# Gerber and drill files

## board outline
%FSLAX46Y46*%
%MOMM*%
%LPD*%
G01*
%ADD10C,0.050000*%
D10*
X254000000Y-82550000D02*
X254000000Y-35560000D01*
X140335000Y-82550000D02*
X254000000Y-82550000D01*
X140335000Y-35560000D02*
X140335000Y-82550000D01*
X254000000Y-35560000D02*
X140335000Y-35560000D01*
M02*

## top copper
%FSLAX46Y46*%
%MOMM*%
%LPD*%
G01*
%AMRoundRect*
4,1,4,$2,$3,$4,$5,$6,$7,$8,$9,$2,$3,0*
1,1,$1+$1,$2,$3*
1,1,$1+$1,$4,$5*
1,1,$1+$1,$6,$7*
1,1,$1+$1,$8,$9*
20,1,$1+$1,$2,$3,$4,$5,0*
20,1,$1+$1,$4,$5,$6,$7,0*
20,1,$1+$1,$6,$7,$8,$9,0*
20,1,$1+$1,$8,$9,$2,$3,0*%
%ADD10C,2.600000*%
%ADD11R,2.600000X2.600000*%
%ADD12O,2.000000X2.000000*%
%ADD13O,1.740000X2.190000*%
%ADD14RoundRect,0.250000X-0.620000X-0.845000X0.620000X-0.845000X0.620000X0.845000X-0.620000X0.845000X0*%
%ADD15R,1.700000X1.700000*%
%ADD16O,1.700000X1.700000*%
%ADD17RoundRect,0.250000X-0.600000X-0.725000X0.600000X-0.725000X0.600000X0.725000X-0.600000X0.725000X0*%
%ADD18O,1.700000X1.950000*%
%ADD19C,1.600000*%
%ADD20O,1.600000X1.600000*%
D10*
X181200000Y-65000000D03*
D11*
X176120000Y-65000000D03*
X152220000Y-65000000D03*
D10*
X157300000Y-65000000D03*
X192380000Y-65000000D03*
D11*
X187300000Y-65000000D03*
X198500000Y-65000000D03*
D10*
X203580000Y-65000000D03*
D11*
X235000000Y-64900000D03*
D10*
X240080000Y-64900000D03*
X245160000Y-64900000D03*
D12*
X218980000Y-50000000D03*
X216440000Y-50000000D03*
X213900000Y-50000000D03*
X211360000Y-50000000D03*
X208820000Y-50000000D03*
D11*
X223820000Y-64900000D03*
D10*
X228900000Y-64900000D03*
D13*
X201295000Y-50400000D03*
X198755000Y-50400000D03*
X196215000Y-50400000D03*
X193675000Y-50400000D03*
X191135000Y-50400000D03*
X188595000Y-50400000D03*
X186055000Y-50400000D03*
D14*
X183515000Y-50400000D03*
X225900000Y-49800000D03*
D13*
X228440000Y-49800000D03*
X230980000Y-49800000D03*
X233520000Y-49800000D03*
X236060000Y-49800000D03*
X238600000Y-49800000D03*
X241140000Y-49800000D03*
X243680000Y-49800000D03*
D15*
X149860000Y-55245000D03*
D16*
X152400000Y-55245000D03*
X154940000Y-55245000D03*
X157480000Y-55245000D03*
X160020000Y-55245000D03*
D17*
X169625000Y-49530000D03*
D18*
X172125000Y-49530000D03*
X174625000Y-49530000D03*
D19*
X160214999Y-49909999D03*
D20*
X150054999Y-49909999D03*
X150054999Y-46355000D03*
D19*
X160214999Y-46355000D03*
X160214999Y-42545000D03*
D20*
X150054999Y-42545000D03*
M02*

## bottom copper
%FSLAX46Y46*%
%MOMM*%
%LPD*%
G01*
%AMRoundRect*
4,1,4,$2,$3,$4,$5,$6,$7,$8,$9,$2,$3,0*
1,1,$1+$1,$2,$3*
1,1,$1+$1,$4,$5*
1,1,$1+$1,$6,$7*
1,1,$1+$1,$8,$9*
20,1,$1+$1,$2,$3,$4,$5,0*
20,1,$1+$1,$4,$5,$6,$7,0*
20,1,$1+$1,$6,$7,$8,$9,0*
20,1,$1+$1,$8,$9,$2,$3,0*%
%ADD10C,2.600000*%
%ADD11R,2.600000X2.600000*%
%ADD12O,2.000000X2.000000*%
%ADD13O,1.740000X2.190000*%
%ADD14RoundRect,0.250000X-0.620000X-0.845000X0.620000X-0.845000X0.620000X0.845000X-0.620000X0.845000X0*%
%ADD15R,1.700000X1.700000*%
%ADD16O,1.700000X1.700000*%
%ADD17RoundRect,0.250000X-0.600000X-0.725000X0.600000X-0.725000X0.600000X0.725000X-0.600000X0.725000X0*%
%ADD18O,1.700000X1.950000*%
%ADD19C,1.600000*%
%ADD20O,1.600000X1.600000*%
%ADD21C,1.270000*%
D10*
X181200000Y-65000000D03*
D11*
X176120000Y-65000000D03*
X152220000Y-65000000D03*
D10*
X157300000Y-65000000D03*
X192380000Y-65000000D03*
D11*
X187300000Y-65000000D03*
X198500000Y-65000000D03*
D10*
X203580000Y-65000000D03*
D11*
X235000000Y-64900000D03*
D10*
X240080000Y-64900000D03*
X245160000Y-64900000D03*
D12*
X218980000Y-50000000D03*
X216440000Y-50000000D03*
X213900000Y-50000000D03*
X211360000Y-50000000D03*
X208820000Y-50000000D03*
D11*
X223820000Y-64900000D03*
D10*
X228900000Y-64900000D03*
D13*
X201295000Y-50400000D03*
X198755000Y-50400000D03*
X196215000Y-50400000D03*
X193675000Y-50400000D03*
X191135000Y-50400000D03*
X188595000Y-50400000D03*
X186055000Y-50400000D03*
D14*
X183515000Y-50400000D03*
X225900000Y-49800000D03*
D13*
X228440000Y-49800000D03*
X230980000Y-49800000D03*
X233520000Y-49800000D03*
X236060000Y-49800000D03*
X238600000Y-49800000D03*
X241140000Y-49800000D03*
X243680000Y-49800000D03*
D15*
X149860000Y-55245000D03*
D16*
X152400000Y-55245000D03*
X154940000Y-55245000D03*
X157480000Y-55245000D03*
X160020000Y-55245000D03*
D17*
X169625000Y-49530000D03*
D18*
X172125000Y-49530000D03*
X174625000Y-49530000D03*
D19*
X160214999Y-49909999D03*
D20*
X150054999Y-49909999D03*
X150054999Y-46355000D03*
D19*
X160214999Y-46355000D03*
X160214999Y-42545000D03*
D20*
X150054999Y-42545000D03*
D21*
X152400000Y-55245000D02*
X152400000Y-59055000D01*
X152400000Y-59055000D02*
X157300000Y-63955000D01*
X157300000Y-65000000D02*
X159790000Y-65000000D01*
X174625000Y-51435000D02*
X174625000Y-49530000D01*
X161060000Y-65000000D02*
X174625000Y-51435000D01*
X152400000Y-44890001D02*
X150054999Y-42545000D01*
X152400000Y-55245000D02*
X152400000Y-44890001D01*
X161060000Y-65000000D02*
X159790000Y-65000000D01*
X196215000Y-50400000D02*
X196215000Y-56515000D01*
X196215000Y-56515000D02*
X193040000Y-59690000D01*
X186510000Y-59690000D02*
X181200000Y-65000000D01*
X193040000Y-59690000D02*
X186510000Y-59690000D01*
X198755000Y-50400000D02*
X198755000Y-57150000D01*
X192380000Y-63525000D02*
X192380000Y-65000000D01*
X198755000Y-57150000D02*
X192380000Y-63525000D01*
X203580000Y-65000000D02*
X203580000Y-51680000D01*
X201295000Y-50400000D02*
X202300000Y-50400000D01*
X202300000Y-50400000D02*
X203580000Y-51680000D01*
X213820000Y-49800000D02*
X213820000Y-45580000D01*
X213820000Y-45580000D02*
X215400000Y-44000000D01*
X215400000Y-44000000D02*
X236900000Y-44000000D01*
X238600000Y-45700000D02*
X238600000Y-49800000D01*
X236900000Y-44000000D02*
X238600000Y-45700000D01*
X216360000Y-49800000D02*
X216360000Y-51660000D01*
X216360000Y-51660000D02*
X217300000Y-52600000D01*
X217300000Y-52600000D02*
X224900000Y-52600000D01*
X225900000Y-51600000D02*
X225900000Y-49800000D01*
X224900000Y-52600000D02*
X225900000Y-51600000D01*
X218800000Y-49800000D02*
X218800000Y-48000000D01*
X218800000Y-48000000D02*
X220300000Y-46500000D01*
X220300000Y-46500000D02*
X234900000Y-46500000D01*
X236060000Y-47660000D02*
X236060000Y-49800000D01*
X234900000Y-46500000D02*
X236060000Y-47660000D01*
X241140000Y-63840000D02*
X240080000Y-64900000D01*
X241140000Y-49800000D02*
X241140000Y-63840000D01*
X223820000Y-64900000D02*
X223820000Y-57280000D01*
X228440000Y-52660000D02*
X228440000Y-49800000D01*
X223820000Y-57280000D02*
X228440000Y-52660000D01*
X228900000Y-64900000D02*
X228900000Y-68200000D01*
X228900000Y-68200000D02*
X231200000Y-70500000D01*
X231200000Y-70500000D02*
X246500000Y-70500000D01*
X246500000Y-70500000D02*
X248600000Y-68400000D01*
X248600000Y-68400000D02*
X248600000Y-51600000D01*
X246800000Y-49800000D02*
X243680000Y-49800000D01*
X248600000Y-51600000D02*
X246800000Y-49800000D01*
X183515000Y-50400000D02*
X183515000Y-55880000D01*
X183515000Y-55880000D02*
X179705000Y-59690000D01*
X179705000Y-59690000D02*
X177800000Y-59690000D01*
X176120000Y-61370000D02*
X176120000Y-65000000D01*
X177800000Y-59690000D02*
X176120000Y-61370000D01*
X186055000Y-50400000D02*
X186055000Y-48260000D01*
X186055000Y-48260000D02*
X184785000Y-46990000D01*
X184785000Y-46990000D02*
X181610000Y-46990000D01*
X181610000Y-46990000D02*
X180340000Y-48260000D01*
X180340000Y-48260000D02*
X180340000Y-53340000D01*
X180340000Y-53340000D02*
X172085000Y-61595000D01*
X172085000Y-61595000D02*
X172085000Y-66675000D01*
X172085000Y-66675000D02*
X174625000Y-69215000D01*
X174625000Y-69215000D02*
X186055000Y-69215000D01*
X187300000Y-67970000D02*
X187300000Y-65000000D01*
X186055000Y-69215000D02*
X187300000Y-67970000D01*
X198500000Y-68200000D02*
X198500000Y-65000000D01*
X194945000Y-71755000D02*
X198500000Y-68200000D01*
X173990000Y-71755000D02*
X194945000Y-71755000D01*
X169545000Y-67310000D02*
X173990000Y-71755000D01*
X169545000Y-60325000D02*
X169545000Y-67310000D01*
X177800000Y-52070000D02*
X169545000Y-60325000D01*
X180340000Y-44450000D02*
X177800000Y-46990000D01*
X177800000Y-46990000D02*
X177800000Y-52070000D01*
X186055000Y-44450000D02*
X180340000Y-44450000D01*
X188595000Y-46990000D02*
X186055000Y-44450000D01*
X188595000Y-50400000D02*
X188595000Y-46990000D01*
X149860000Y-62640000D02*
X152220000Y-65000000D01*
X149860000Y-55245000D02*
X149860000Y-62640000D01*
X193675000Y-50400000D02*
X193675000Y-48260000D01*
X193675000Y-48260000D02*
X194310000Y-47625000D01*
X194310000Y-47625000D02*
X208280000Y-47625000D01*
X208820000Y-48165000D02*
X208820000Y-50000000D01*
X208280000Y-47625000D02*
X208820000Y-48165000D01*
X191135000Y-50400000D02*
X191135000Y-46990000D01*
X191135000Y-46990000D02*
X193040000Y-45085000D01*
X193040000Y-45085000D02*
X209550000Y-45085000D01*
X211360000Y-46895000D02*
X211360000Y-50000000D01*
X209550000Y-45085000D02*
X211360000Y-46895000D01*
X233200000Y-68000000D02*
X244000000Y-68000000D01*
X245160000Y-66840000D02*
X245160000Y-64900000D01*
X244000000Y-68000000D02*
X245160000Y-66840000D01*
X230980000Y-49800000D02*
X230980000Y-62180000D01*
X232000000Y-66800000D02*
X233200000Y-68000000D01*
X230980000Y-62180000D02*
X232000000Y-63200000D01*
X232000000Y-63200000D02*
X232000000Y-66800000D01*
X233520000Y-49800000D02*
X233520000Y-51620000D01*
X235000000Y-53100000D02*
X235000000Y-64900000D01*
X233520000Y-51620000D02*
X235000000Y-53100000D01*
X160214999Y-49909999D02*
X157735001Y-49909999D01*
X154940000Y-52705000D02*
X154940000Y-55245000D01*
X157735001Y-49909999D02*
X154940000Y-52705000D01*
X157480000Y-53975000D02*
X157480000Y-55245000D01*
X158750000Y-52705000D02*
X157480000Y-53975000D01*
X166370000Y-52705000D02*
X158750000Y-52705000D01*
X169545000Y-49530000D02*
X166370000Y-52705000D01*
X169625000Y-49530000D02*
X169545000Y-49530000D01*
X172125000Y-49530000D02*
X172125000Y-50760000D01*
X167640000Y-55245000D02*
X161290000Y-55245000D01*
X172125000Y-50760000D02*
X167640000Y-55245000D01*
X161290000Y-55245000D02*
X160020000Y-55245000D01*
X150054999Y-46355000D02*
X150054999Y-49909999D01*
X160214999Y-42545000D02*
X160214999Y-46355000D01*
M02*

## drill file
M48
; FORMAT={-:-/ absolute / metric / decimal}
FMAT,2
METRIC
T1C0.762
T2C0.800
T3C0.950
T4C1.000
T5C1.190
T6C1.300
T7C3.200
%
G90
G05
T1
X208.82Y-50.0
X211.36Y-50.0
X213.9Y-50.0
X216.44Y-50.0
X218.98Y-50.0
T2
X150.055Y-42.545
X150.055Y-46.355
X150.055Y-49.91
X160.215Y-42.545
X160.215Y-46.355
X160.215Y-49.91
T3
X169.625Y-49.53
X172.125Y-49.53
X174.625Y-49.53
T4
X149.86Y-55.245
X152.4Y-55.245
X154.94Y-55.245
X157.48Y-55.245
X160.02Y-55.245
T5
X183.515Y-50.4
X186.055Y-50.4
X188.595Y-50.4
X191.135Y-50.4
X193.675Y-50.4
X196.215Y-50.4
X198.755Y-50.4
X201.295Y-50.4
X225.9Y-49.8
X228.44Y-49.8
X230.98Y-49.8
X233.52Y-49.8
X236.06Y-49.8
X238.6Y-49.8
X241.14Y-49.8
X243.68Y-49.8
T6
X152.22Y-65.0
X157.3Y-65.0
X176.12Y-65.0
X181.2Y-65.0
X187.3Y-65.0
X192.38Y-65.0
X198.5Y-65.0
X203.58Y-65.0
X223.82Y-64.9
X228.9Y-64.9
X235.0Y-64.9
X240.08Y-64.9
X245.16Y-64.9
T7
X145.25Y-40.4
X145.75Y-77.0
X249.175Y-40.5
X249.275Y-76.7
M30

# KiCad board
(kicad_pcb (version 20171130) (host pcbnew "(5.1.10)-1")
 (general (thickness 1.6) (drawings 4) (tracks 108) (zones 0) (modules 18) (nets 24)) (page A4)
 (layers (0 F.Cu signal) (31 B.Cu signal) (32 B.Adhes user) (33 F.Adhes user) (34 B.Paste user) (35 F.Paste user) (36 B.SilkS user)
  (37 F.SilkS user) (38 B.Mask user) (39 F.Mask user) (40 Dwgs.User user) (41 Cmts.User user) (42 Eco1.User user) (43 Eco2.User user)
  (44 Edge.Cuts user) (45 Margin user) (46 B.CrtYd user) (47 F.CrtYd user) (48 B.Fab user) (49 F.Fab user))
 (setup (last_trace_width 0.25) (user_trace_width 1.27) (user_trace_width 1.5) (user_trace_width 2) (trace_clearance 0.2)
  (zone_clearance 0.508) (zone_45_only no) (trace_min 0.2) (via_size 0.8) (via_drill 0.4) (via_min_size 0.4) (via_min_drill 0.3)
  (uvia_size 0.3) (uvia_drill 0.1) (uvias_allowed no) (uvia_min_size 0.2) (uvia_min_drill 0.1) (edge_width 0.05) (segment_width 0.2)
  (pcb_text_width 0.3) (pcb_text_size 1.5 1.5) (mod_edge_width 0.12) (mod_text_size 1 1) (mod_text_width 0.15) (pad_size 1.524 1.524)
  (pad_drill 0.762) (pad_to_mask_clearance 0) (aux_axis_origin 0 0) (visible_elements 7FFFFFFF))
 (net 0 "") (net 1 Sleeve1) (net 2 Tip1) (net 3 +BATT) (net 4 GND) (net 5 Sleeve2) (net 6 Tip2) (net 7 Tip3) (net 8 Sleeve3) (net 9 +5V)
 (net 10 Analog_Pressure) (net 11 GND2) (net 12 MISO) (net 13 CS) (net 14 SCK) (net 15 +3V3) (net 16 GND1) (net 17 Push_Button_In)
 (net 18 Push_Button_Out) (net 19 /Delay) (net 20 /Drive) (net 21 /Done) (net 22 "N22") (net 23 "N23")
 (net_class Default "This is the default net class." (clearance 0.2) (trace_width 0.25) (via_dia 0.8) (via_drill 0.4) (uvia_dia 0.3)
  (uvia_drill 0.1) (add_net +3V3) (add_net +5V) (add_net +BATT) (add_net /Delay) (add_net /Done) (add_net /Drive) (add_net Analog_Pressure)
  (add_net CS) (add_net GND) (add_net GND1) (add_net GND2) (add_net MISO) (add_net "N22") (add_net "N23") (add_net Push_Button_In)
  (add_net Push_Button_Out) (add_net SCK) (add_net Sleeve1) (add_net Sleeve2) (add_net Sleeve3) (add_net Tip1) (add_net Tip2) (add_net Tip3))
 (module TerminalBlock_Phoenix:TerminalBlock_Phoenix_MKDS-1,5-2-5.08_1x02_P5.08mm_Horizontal (layer F.Cu) (at 176.12 65)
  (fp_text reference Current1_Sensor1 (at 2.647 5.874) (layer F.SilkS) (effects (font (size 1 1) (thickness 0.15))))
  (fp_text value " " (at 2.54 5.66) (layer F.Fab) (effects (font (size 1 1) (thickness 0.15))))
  (pad 2 thru_hole circle (at 5.08 0) (size 2.6 2.6) (drill 1.3) (layers *.Cu *.Mask) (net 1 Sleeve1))
  (pad 1 thru_hole rect (at 0 0) (size 2.6 2.6) (drill 1.3) (layers *.Cu *.Mask) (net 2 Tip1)))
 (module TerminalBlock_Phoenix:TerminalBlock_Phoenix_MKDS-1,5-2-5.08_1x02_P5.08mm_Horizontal (layer F.Cu) (at 152.22 65)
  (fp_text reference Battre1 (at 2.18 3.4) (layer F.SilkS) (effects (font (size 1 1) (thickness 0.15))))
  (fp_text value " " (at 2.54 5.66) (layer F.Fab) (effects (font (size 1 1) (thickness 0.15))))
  (pad 1 thru_hole rect (at 0 0) (size 2.6 2.6) (drill 1.3) (layers *.Cu *.Mask) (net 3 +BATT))
  (pad 2 thru_hole circle (at 5.08 0) (size 2.6 2.6) (drill 1.3) (layers *.Cu *.Mask) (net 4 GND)))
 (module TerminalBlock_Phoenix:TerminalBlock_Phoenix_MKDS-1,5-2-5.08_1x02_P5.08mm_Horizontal (layer F.Cu) (at 187.3 65)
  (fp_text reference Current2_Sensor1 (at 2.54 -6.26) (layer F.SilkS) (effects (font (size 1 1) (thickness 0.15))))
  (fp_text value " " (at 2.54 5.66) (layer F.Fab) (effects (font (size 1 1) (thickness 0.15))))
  (pad 2 thru_hole circle (at 5.08 0) (size 2.6 2.6) (drill 1.3) (layers *.Cu *.Mask) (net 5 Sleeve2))
  (pad 1 thru_hole rect (at 0 0) (size 2.6 2.6) (drill 1.3) (layers *.Cu *.Mask) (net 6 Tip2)))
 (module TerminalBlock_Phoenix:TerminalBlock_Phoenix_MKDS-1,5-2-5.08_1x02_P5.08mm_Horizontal (layer F.Cu) (at 198.5 65)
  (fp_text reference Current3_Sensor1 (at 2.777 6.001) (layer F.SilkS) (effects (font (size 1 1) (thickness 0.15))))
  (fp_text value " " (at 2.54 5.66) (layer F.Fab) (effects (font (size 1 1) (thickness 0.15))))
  (pad 1 thru_hole rect (at 0 0) (size 2.6 2.6) (drill 1.3) (layers *.Cu *.Mask) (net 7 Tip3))
  (pad 2 thru_hole circle (at 5.08 0) (size 2.6 2.6) (drill 1.3) (layers *.Cu *.Mask) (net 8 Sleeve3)))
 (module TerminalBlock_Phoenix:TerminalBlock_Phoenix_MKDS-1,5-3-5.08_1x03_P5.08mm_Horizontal (layer F.Cu) (at 235 64.9)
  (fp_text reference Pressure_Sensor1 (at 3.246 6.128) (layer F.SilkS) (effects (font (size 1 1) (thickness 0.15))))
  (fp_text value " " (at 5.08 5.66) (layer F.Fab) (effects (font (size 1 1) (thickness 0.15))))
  (pad 1 thru_hole rect (at 0 0) (size 2.6 2.6) (drill 1.3) (layers *.Cu *.Mask) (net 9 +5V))
  (pad 2 thru_hole circle (at 5.08 0) (size 2.6 2.6) (drill 1.3) (layers *.Cu *.Mask) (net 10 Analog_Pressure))
  (pad 3 thru_hole circle (at 10.16 0) (size 2.6 2.6) (drill 1.3) (layers *.Cu *.Mask) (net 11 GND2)))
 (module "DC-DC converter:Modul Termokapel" (layer F.Cu) (at 213.9 55.08)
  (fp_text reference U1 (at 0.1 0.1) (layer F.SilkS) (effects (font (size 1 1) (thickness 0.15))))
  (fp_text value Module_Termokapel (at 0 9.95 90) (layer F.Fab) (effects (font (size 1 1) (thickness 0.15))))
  (pad 5 thru_hole oval (at 5.08 -5.08) (size 2 2) (drill 0.762) (layers *.Cu *.Mask) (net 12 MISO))
  (pad 4 thru_hole oval (at 2.54 -5.08) (size 2 2) (drill 0.762) (layers *.Cu *.Mask) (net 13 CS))
  (pad 3 thru_hole oval (at 0 -5.08) (size 2 2) (drill 0.762) (layers *.Cu *.Mask) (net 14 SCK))
  (pad 2 thru_hole oval (at -2.54 -5.08) (size 2 2) (drill 0.762) (layers *.Cu *.Mask) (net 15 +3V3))
  (pad 1 thru_hole oval (at -5.08 -5.08) (size 2 2) (drill 0.762) (layers *.Cu *.Mask) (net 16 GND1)))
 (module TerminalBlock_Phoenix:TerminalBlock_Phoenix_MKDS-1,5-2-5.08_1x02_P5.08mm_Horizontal (layer F.Cu) (at 223.82 64.9)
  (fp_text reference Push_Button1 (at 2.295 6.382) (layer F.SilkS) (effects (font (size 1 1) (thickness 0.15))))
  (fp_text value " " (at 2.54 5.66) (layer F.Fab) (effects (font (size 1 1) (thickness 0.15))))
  (pad 1 thru_hole rect (at 0 0) (size 2.6 2.6) (drill 1.3) (layers *.Cu *.Mask) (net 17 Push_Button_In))
  (pad 2 thru_hole circle (at 5.08 0) (size 2.6 2.6) (drill 1.3) (layers *.Cu *.Mask) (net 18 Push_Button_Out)))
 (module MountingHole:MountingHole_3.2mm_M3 (layer F.Cu) (at 145.75 77)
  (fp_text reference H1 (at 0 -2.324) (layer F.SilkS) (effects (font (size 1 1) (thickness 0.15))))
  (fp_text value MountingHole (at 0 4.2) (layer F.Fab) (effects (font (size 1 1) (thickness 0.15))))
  (pad 1 np_thru_hole circle (at 0 0) (size 3.2 3.2) (drill 3.2) (layers *.Cu *.Mask)))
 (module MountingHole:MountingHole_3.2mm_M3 (layer F.Cu) (at 145.25 40.4)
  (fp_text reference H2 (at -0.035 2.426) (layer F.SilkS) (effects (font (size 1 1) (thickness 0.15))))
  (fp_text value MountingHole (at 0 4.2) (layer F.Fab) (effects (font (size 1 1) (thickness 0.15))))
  (pad 1 np_thru_hole circle (at 0 0) (size 3.2 3.2) (drill 3.2) (layers *.Cu *.Mask)))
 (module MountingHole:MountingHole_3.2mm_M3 (layer F.Cu) (at 249.275 76.7)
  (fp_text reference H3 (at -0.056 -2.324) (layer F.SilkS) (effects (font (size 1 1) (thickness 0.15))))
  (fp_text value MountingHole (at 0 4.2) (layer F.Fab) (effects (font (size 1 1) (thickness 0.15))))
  (pad 1 np_thru_hole circle (at 0 0) (size 3.2 3.2) (drill 3.2) (layers *.Cu *.Mask)))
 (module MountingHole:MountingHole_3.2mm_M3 (layer F.Cu) (at 249.175 40.5)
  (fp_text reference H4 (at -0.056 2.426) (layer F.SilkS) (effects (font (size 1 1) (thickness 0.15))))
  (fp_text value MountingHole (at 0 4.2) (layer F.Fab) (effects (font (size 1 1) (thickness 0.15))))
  (pad 1 np_thru_hole circle (at 0 0) (size 3.2 3.2) (drill 3.2) (layers *.Cu *.Mask)))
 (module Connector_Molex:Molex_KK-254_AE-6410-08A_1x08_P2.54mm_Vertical (layer F.Cu) (at 183.515 50.4)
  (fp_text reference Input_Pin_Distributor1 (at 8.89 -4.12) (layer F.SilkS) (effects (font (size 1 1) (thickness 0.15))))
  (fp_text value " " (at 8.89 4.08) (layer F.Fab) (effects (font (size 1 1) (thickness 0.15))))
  (pad 8 thru_hole oval (at 17.78 0) (size 1.74 2.19) (drill 1.19) (layers *.Cu *.Mask) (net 8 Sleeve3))
  (pad 7 thru_hole oval (at 15.24 0) (size 1.74 2.19) (drill 1.19) (layers *.Cu *.Mask) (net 5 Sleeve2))
  (pad 6 thru_hole oval (at 12.7 0) (size 1.74 2.19) (drill 1.19) (layers *.Cu *.Mask) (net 1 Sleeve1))
  (pad 5 thru_hole oval (at 10.16 0) (size 1.74 2.19) (drill 1.19) (layers *.Cu *.Mask) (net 16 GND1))
  (pad 4 thru_hole oval (at 7.62 0) (size 1.74 2.19) (drill 1.19) (layers *.Cu *.Mask) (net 15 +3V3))
  (pad 3 thru_hole oval (at 5.08 0) (size 1.74 2.19) (drill 1.19) (layers *.Cu *.Mask) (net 7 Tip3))
  (pad 2 thru_hole oval (at 2.54 0) (size 1.74 2.19) (drill 1.19) (layers *.Cu *.Mask) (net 6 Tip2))
  (pad 1 thru_hole roundrect (at 0 0) (size 1.74 2.19) (drill 1.19) (layers *.Cu *.Mask) (roundrect_rratio 0.143678) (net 2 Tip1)))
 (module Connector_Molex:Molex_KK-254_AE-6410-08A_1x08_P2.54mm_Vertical (layer F.Cu) (at 225.9 49.8)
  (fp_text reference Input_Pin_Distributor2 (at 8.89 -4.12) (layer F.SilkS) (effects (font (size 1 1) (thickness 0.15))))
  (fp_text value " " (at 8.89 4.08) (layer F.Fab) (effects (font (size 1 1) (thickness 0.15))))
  (pad 1 thru_hole roundrect (at 0 0) (size 1.74 2.19) (drill 1.19) (layers *.Cu *.Mask) (roundrect_rratio 0.143678) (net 13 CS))
  (pad 2 thru_hole oval (at 2.54 0) (size 1.74 2.19) (drill 1.19) (layers *.Cu *.Mask) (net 17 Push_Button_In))
  (pad 3 thru_hole oval (at 5.08 0) (size 1.74 2.19) (drill 1.19) (layers *.Cu *.Mask) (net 11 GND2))
  (pad 4 thru_hole oval (at 7.62 0) (size 1.74 2.19) (drill 1.19) (layers *.Cu *.Mask) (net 9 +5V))
  (pad 5 thru_hole oval (at 10.16 0) (size 1.74 2.19) (drill 1.19) (layers *.Cu *.Mask) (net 12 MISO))
  (pad 6 thru_hole oval (at 12.7 0) (size 1.74 2.19) (drill 1.19) (layers *.Cu *.Mask) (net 14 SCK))
  (pad 7 thru_hole oval (at 15.24 0) (size 1.74 2.19) (drill 1.19) (layers *.Cu *.Mask) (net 10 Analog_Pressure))
  (pad 8 thru_hole oval (at 17.78 0) (size 1.74 2.19) (drill 1.19) (layers *.Cu *.Mask) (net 18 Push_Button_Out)))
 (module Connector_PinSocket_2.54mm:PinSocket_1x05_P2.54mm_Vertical (layer F.Cu) (at 149.86 55.245 90)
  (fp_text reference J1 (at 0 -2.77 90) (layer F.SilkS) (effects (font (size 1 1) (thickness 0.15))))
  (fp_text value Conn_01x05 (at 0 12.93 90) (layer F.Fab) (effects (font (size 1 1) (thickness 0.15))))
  (pad 1 thru_hole rect (at 0 0 90) (size 1.7 1.7) (drill 1) (layers *.Cu *.Mask) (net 3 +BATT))
  (pad 2 thru_hole oval (at 0 2.54 90) (size 1.7 1.7) (drill 1) (layers *.Cu *.Mask) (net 4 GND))
  (pad 3 thru_hole oval (at 0 5.08 90) (size 1.7 1.7) (drill 1) (layers *.Cu *.Mask) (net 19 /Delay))
  (pad 4 thru_hole oval (at 0 7.62 90) (size 1.7 1.7) (drill 1) (layers *.Cu *.Mask) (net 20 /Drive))
  (pad 5 thru_hole oval (at 0 10.16 90) (size 1.7 1.7) (drill 1) (layers *.Cu *.Mask) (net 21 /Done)))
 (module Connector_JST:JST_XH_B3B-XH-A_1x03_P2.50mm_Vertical (layer F.Cu) (at 169.625 49.53)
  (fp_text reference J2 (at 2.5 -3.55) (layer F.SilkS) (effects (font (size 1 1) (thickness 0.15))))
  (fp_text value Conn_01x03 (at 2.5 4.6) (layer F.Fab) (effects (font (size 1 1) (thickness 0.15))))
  (pad 1 thru_hole roundrect (at 0 0) (size 1.7 1.95) (drill 0.95) (layers *.Cu *.Mask) (roundrect_rratio 0.147059) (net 20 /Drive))
  (pad 2 thru_hole oval (at 2.5 0) (size 1.7 1.95) (drill 0.95) (layers *.Cu *.Mask) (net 21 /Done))
  (pad 3 thru_hole oval (at 5 0) (size 1.7 1.95) (drill 0.95) (layers *.Cu *.Mask) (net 4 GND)))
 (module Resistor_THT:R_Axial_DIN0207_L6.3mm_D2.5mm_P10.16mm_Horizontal (layer F.Cu) (at 160.214999 49.909999 180)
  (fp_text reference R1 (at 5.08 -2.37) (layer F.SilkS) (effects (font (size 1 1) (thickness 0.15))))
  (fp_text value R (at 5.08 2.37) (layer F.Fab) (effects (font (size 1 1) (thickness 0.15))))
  (pad 1 thru_hole circle (at 0 0 180) (size 1.6 1.6) (drill 0.8) (layers *.Cu *.Mask) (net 19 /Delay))
  (pad 2 thru_hole oval (at 10.16 0 180) (size 1.6 1.6) (drill 0.8) (layers *.Cu *.Mask) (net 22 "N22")))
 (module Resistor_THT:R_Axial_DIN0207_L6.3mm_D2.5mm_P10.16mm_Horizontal (layer F.Cu) (at 160.214999 46.355 180)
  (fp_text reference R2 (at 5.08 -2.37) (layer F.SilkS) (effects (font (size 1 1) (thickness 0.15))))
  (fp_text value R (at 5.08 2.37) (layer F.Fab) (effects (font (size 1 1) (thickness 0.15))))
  (pad 2 thru_hole oval (at 10.16 0 180) (size 1.6 1.6) (drill 0.8) (layers *.Cu *.Mask) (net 22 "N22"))
  (pad 1 thru_hole circle (at 0 0 180) (size 1.6 1.6) (drill 0.8) (layers *.Cu *.Mask) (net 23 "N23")))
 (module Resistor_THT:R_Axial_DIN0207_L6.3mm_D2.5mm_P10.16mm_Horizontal (layer F.Cu) (at 160.214999 42.545 180)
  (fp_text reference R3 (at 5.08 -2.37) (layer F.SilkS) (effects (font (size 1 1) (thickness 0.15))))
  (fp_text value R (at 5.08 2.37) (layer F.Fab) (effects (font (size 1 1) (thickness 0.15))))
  (pad 1 thru_hole circle (at 0 0 180) (size 1.6 1.6) (drill 0.8) (layers *.Cu *.Mask) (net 23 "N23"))
  (pad 2 thru_hole oval (at 10.16 0 180) (size 1.6 1.6) (drill 0.8) (layers *.Cu *.Mask) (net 4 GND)))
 (gr_line (start 254 82.55) (end 254 35.56) (layer Edge.Cuts) (width 0.05))
 (gr_line (start 140.335 82.55) (end 254 82.55) (layer Edge.Cuts) (width 0.05))
 (gr_line (start 140.335 35.56) (end 140.335 82.55) (layer Edge.Cuts) (width 0.05))
 (gr_line (start 254 35.56) (end 140.335 35.56) (layer Edge.Cuts) (width 0.05))
 (segment (start 152.4 55.245) (end 152.4 59.055) (width 1.27) (layer B.Cu) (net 4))
 (segment (start 152.4 59.055) (end 157.3 63.955) (width 1.27) (layer B.Cu) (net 4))
 (segment (start 157.3 65) (end 159.79 65) (width 1.27) (layer B.Cu) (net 4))
 (segment (start 174.625 51.435) (end 174.625 49.53) (width 1.27) (layer B.Cu) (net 4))
 (segment (start 161.06 65) (end 174.625 51.435) (width 1.27) (layer B.Cu) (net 4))
 (segment (start 152.4 44.890001) (end 150.054999 42.545) (width 1.27) (layer B.Cu) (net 4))
 (segment (start 152.4 55.245) (end 152.4 44.890001) (width 1.27) (layer B.Cu) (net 4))
 (segment (start 161.06 65) (end 159.79 65) (width 1.27) (layer B.Cu) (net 4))
 (segment (start 196.215 50.4) (end 196.215 56.515) (width 1.27) (layer B.Cu) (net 1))
 (segment (start 196.215 56.515) (end 193.04 59.69) (width 1.27) (layer B.Cu) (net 1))
 (segment (start 186.51 59.69) (end 181.2 65) (width 1.27) (layer B.Cu) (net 1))
 (segment (start 193.04 59.69) (end 186.51 59.69) (width 1.27) (layer B.Cu) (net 1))
 (segment (start 198.755 50.4) (end 198.755 57.15) (width 1.27) (layer B.Cu) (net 5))
 (segment (start 192.38 63.525) (end 192.38 65) (width 1.27) (layer B.Cu) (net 5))
 (segment (start 198.755 57.15) (end 192.38 63.525) (width 1.27) (layer B.Cu) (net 5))
 (segment (start 203.58 65) (end 203.58 51.68) (width 1.27) (layer B.Cu) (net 8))
 (segment (start 201.295 50.4) (end 202.3 50.4) (width 1.27) (layer B.Cu) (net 8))
 (segment (start 202.3 50.4) (end 203.58 51.68) (width 1.27) (layer B.Cu) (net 8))
 (segment (start 213.82 49.8) (end 213.82 45.58) (width 1.27) (layer B.Cu) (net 14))
 (segment (start 213.82 45.58) (end 215.4 44) (width 1.27) (layer B.Cu) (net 14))
 (segment (start 215.4 44) (end 236.9 44) (width 1.27) (layer B.Cu) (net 14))
 (segment (start 238.6 45.7) (end 238.6 49.8) (width 1.27) (layer B.Cu) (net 14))
 (segment (start 236.9 44) (end 238.6 45.7) (width 1.27) (layer B.Cu) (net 14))
 (segment (start 216.36 49.8) (end 216.36 51.66) (width 1.27) (layer B.Cu) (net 13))
 (segment (start 216.36 51.66) (end 217.3 52.6) (width 1.27) (layer B.Cu) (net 13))
 (segment (start 217.3 52.6) (end 224.9 52.6) (width 1.27) (layer B.Cu) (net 13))
 (segment (start 225.9 51.6) (end 225.9 49.8) (width 1.27) (layer B.Cu) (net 13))
 (segment (start 224.9 52.6) (end 225.9 51.6) (width 1.27) (layer B.Cu) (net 13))
 (segment (start 218.8 49.8) (end 218.8 48) (width 1.27) (layer B.Cu) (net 12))
 (segment (start 218.8 48) (end 220.3 46.5) (width 1.27) (layer B.Cu) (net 12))
 (segment (start 220.3 46.5) (end 234.9 46.5) (width 1.27) (layer B.Cu) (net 12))
 (segment (start 236.06 47.66) (end 236.06 49.8) (width 1.27) (layer B.Cu) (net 12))
 (segment (start 234.9 46.5) (end 236.06 47.66) (width 1.27) (layer B.Cu) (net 12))
 (segment (start 241.14 63.84) (end 240.08 64.9) (width 1.27) (layer B.Cu) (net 10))
 (segment (start 241.14 49.8) (end 241.14 63.84) (width 1.27) (layer B.Cu) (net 10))
 (segment (start 223.82 64.9) (end 223.82 57.28) (width 1.27) (layer B.Cu) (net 17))
 (segment (start 228.44 52.66) (end 228.44 49.8) (width 1.27) (layer B.Cu) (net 17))
 (segment (start 223.82 57.28) (end 228.44 52.66) (width 1.27) (layer B.Cu) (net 17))
 (segment (start 228.9 64.9) (end 228.9 68.2) (width 1.27) (layer B.Cu) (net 18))
 (segment (start 228.9 68.2) (end 231.2 70.5) (width 1.27) (layer B.Cu) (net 18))
 (segment (start 231.2 70.5) (end 246.5 70.5) (width 1.27) (layer B.Cu) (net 18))
 (segment (start 246.5 70.5) (end 248.6 68.4) (width 1.27) (layer B.Cu) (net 18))
 (segment (start 248.6 68.4) (end 248.6 51.6) (width 1.27) (layer B.Cu) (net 18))
 (segment (start 246.8 49.8) (end 243.68 49.8) (width 1.27) (layer B.Cu) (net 18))
 (segment (start 248.6 51.6) (end 246.8 49.8) (width 1.27) (layer B.Cu) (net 18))
 (segment (start 183.515 50.4) (end 183.515 55.88) (width 1.27) (layer B.Cu) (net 2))
 (segment (start 183.515 55.88) (end 179.705 59.69) (width 1.27) (layer B.Cu) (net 2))
 (segment (start 179.705 59.69) (end 177.8 59.69) (width 1.27) (layer B.Cu) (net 2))
 (segment (start 176.12 61.37) (end 176.12 65) (width 1.27) (layer B.Cu) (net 2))
 (segment (start 177.8 59.69) (end 176.12 61.37) (width 1.27) (layer B.Cu) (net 2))
 (segment (start 186.055 50.4) (end 186.055 48.26) (width 1.27) (layer B.Cu) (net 6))
 (segment (start 186.055 48.26) (end 184.785 46.99) (width 1.27) (layer B.Cu) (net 6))
 (segment (start 184.785 46.99) (end 181.61 46.99) (width 1.27) (layer B.Cu) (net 6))
 (segment (start 181.61 46.99) (end 180.34 48.26) (width 1.27) (layer B.Cu) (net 6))
 (segment (start 180.34 48.26) (end 180.34 53.34) (width 1.27) (layer B.Cu) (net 6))
 (segment (start 180.34 53.34) (end 172.085 61.595) (width 1.27) (layer B.Cu) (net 6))
 (segment (start 172.085 61.595) (end 172.085 66.675) (width 1.27) (layer B.Cu) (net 6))
 (segment (start 172.085 66.675) (end 174.625 69.215) (width 1.27) (layer B.Cu) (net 6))
 (segment (start 174.625 69.215) (end 186.055 69.215) (width 1.27) (layer B.Cu) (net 6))
 (segment (start 187.3 67.97) (end 187.3 65) (width 1.27) (layer B.Cu) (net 6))
 (segment (start 186.055 69.215) (end 187.3 67.97) (width 1.27) (layer B.Cu) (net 6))
 (segment (start 198.5 68.2) (end 198.5 65) (width 1.27) (layer B.Cu) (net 7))
 (segment (start 194.945 71.755) (end 198.5 68.2) (width 1.27) (layer B.Cu) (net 7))
 (segment (start 173.99 71.755) (end 194.945 71.755) (width 1.27) (layer B.Cu) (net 7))
 (segment (start 169.545 67.31) (end 173.99 71.755) (width 1.27) (layer B.Cu) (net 7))
 (segment (start 169.545 60.325) (end 169.545 67.31) (width 1.27) (layer B.Cu) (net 7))
 (segment (start 177.8 52.07) (end 169.545 60.325) (width 1.27) (layer B.Cu) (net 7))
 (segment (start 180.34 44.45) (end 177.8 46.99) (width 1.27) (layer B.Cu) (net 7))
 (segment (start 177.8 46.99) (end 177.8 52.07) (width 1.27) (layer B.Cu) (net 7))
 (segment (start 186.055 44.45) (end 180.34 44.45) (width 1.27) (layer B.Cu) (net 7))
 (segment (start 188.595 46.99) (end 186.055 44.45) (width 1.27) (layer B.Cu) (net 7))
 (segment (start 188.595 50.4) (end 188.595 46.99) (width 1.27) (layer B.Cu) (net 7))
 (segment (start 149.86 62.64) (end 152.22 65) (width 1.27) (layer B.Cu) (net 3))
 (segment (start 149.86 55.245) (end 149.86 62.64) (width 1.27) (layer B.Cu) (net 3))
 (segment (start 193.675 50.4) (end 193.675 48.26) (width 1.27) (layer B.Cu) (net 16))
 (segment (start 193.675 48.26) (end 194.31 47.625) (width 1.27) (layer B.Cu) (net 16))
 (segment (start 194.31 47.625) (end 208.28 47.625) (width 1.27) (layer B.Cu) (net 16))
 (segment (start 208.82 48.165) (end 208.82 50) (width 1.27) (layer B.Cu) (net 16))
 (segment (start 208.28 47.625) (end 208.82 48.165) (width 1.27) (layer B.Cu) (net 16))
 (segment (start 191.135 50.4) (end 191.135 46.99) (width 1.27) (layer B.Cu) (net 15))
 (segment (start 191.135 46.99) (end 193.04 45.085) (width 1.27) (layer B.Cu) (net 15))
 (segment (start 193.04 45.085) (end 209.55 45.085) (width 1.27) (layer B.Cu) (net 15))
 (segment (start 211.36 46.895) (end 211.36 50) (width 1.27) (layer B.Cu) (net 15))
 (segment (start 209.55 45.085) (end 211.36 46.895) (width 1.27) (layer B.Cu) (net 15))
 (segment (start 233.2 68) (end 244 68) (width 1.27) (layer B.Cu) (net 11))
 (segment (start 245.16 66.84) (end 245.16 64.9) (width 1.27) (layer B.Cu) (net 11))
 (segment (start 244 68) (end 245.16 66.84) (width 1.27) (layer B.Cu) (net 11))
 (segment (start 230.98 49.8) (end 230.98 62.18) (width 1.27) (layer B.Cu) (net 11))
 (segment (start 232 66.8) (end 233.2 68) (width 1.27) (layer B.Cu) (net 11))
 (segment (start 230.98 62.18) (end 232 63.2) (width 1.27) (layer B.Cu) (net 11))
 (segment (start 232 63.2) (end 232 66.8) (width 1.27) (layer B.Cu) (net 11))
 (segment (start 233.52 49.8) (end 233.52 51.62) (width 1.27) (layer B.Cu) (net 9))
 (segment (start 235 53.1) (end 235 64.9) (width 1.27) (layer B.Cu) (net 9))
 (segment (start 233.52 51.62) (end 235 53.1) (width 1.27) (layer B.Cu) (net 9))
 (segment (start 160.214999 49.909999) (end 157.735001 49.909999) (width 1.27) (layer B.Cu) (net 19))
 (segment (start 154.94 52.705) (end 154.94 55.245) (width 1.27) (layer B.Cu) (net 19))
 (segment (start 157.735001 49.909999) (end 154.94 52.705) (width 1.27) (layer B.Cu) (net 19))
 (segment (start 157.48 53.975) (end 157.48 55.245) (width 1.27) (layer B.Cu) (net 20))
 (segment (start 158.75 52.705) (end 157.48 53.975) (width 1.27) (layer B.Cu) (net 20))
 (segment (start 166.37 52.705) (end 158.75 52.705) (width 1.27) (layer B.Cu) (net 20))
 (segment (start 169.545 49.53) (end 166.37 52.705) (width 1.27) (layer B.Cu) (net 20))
 (segment (start 169.625 49.53) (end 169.545 49.53) (width 1.27) (layer B.Cu) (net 20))
 (segment (start 172.125 49.53) (end 172.125 50.76) (width 1.27) (layer B.Cu) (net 21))
 (segment (start 167.64 55.245) (end 161.29 55.245) (width 1.27) (layer B.Cu) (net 21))
 (segment (start 172.125 50.76) (end 167.64 55.245) (width 1.27) (layer B.Cu) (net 21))
 (segment (start 161.29 55.245) (end 160.02 55.245) (width 1.27) (layer B.Cu) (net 21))
 (segment (start 150.054999 46.355) (end 150.054999 49.909999) (width 1.27) (layer B.Cu) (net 22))
 (segment (start 160.214999 42.545) (end 160.214999 46.355) (width 1.27) (layer B.Cu) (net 23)))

